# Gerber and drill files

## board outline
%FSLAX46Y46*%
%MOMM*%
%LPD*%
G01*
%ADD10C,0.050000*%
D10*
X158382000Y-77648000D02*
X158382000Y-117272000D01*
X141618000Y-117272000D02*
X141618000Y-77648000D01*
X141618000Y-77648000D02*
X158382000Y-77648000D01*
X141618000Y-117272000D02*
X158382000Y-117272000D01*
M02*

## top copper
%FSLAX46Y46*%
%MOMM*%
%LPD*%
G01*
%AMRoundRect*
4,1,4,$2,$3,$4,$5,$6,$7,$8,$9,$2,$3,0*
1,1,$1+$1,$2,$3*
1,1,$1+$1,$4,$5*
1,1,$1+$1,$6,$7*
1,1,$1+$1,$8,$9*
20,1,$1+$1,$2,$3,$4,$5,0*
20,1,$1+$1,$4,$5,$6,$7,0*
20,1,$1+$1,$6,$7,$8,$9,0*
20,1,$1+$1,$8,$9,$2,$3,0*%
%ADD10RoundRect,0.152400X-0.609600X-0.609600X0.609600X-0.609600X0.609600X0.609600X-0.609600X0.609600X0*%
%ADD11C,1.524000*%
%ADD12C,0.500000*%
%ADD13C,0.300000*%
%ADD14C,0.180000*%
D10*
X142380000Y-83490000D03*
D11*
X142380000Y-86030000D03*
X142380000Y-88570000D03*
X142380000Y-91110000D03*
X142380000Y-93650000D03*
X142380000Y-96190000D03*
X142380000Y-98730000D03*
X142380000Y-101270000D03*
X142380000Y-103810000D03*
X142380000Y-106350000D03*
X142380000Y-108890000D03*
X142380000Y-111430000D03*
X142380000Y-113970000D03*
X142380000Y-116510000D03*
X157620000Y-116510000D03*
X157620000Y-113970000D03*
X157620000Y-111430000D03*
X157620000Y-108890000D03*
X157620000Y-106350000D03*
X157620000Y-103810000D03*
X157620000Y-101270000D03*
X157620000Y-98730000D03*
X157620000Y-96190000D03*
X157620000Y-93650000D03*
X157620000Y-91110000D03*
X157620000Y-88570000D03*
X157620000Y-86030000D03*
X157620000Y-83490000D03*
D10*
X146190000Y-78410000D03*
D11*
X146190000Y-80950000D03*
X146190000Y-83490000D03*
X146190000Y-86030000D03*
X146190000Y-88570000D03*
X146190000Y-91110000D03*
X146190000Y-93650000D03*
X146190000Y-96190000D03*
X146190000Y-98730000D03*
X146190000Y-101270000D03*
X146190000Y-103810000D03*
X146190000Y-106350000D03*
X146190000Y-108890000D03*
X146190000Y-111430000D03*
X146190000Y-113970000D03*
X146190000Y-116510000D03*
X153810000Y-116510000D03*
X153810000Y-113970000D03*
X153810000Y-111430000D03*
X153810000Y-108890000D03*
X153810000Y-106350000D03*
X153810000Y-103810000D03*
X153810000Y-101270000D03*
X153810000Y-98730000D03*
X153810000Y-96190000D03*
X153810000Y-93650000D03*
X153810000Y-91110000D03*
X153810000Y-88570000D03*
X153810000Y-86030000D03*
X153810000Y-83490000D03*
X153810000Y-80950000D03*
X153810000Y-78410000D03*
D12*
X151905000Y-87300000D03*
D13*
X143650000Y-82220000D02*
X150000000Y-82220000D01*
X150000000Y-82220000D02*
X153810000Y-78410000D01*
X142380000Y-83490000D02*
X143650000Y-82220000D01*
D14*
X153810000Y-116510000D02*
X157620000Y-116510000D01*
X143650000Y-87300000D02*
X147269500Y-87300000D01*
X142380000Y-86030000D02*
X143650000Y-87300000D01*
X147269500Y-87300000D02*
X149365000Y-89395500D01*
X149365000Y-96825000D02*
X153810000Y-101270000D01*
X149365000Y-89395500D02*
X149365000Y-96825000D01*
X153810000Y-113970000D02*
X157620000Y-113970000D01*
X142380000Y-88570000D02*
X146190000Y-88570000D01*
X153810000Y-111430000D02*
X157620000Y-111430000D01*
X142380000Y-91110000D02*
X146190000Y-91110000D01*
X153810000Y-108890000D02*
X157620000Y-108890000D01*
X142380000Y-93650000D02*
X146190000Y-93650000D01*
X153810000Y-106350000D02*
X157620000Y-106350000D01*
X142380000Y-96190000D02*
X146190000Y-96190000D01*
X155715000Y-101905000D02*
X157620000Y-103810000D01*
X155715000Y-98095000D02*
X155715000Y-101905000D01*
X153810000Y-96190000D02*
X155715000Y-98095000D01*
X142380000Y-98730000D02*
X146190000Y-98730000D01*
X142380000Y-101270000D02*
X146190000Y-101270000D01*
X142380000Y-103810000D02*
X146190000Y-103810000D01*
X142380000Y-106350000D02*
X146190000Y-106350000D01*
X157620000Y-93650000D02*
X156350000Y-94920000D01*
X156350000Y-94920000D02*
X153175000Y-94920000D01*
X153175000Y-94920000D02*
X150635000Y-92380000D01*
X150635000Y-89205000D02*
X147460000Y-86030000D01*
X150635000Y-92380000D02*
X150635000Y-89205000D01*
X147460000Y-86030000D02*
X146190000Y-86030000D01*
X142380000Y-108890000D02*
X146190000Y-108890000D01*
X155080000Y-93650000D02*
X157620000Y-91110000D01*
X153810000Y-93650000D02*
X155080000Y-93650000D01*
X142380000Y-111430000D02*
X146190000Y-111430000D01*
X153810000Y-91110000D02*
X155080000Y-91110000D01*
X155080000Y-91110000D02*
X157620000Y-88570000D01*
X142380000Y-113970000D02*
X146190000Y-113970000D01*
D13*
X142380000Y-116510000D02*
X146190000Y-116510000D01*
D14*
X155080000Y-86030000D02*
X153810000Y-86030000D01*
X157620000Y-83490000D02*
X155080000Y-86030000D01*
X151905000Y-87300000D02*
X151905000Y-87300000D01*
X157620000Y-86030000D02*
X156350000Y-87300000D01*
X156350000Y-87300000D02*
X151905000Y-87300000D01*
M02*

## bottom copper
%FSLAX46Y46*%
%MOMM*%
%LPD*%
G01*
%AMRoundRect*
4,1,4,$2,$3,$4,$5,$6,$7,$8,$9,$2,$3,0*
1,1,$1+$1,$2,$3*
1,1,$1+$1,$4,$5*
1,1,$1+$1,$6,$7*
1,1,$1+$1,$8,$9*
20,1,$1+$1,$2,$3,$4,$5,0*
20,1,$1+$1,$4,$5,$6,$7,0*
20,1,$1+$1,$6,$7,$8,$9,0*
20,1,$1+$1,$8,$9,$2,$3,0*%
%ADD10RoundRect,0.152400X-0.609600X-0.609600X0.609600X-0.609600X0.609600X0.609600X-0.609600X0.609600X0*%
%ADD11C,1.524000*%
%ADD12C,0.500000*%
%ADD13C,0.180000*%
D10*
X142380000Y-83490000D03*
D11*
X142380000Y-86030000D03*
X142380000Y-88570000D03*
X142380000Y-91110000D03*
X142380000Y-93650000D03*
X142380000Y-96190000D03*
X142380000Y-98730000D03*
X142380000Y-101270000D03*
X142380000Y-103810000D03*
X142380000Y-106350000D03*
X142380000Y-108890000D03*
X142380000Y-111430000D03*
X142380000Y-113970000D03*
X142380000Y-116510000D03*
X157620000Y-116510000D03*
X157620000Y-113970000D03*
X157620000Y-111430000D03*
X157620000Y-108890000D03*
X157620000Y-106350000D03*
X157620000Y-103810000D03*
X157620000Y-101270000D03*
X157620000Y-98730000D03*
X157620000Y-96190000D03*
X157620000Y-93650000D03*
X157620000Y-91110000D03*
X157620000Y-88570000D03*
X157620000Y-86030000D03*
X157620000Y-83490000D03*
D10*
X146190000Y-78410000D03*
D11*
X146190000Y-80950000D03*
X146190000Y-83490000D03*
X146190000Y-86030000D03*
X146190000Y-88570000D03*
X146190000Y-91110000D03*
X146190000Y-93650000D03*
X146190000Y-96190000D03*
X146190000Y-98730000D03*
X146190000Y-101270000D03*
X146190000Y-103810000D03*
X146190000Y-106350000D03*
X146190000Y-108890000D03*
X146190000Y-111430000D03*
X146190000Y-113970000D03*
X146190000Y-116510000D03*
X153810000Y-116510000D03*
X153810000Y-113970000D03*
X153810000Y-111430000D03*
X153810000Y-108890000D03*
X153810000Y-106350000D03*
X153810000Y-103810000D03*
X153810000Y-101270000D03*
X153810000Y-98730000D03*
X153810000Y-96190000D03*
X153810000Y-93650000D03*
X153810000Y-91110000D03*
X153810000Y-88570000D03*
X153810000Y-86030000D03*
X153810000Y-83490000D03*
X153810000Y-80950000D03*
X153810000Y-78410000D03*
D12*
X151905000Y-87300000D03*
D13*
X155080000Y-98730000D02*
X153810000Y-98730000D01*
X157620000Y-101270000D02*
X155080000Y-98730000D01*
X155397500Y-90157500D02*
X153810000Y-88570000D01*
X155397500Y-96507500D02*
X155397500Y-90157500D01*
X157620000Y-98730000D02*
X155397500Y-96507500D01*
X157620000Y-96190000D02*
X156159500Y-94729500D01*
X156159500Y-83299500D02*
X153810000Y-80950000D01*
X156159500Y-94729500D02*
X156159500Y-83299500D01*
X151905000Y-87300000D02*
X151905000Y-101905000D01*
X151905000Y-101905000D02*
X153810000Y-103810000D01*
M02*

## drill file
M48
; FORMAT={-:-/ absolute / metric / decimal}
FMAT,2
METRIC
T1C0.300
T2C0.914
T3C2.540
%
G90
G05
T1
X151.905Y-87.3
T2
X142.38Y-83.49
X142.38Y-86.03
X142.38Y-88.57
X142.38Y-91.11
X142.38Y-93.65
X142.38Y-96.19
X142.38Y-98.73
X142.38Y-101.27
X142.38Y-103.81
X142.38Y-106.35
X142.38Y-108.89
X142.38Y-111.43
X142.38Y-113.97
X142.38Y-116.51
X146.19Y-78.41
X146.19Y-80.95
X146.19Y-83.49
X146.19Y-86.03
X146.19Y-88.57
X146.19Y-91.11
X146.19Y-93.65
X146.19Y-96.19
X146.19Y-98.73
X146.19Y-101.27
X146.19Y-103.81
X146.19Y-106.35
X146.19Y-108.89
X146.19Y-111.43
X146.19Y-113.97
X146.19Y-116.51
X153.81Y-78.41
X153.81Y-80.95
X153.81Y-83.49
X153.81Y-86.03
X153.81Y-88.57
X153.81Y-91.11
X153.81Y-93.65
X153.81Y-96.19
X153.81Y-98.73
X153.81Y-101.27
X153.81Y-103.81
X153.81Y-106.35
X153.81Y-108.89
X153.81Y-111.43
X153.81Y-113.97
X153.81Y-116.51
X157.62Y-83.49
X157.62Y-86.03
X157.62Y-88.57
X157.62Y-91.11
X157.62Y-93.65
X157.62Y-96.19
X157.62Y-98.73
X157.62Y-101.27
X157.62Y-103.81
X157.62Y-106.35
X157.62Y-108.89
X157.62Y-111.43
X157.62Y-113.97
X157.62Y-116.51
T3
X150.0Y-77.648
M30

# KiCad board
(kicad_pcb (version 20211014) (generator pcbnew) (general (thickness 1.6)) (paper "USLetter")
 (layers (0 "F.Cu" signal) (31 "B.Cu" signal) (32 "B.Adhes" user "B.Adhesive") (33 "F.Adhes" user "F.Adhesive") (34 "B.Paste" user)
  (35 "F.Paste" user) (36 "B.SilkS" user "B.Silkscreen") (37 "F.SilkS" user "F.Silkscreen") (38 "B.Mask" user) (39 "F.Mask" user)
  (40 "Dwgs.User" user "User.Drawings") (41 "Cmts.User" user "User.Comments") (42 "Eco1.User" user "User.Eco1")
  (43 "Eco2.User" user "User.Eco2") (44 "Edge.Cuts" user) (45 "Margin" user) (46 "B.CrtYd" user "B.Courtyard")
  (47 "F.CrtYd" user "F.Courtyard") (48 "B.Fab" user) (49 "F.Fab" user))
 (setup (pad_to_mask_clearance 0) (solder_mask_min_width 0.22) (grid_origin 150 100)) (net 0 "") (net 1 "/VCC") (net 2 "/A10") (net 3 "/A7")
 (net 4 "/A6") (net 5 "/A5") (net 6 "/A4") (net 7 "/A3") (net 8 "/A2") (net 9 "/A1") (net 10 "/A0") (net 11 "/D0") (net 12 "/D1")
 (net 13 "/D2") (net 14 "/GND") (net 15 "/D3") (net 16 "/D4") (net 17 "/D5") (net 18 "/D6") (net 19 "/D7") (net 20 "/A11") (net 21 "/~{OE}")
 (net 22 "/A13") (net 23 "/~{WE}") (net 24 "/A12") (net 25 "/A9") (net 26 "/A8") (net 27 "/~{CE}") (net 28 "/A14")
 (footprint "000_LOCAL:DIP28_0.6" (layer "F.Cu") (at 150 100)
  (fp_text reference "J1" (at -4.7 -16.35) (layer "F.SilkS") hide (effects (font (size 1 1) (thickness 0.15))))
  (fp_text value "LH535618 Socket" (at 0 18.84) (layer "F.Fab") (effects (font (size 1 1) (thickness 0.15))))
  (pad "1" thru_hole roundrect locked (at -7.62 -16.51) (size 1.524 1.524) (drill 0.9144) (layers *.Cu *.Mask) (roundrect_rratio 0.1)
   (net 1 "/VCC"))
  (pad "2" thru_hole circle locked (at -7.62 -13.97) (size 1.524 1.524) (drill 0.9144) (layers *.Cu *.Mask) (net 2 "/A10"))
  (pad "3" thru_hole circle locked (at -7.62 -11.43) (size 1.524 1.524) (drill 0.9144) (layers *.Cu *.Mask) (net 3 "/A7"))
  (pad "4" thru_hole circle locked (at -7.62 -8.89) (size 1.524 1.524) (drill 0.9144) (layers *.Cu *.Mask) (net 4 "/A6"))
  (pad "5" thru_hole circle locked (at -7.62 -6.35) (size 1.524 1.524) (drill 0.9144) (layers *.Cu *.Mask) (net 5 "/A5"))
  (pad "6" thru_hole circle locked (at -7.62 -3.81) (size 1.524 1.524) (drill 0.9144) (layers *.Cu *.Mask) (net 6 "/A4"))
  (pad "7" thru_hole circle locked (at -7.62 -1.27) (size 1.524 1.524) (drill 0.9144) (layers *.Cu *.Mask) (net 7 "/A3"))
  (pad "8" thru_hole circle locked (at -7.62 1.27) (size 1.524 1.524) (drill 0.9144) (layers *.Cu *.Mask) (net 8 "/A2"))
  (pad "9" thru_hole circle locked (at -7.62 3.81) (size 1.524 1.524) (drill 0.9144) (layers *.Cu *.Mask) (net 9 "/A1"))
  (pad "10" thru_hole circle locked (at -7.62 6.35) (size 1.524 1.524) (drill 0.9144) (layers *.Cu *.Mask) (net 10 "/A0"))
  (pad "11" thru_hole circle locked (at -7.62 8.89) (size 1.524 1.524) (drill 0.9144) (layers *.Cu *.Mask) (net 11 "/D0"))
  (pad "12" thru_hole circle locked (at -7.62 11.43) (size 1.524 1.524) (drill 0.9144) (layers *.Cu *.Mask) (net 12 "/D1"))
  (pad "13" thru_hole circle locked (at -7.62 13.97) (size 1.524 1.524) (drill 0.9144) (layers *.Cu *.Mask) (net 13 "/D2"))
  (pad "14" thru_hole circle locked (at -7.62 16.51) (size 1.524 1.524) (drill 0.9144) (layers *.Cu *.Mask) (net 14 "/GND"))
  (pad "15" thru_hole circle locked (at 7.62 16.51) (size 1.524 1.524) (drill 0.9144) (layers *.Cu *.Mask) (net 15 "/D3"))
  (pad "16" thru_hole circle locked (at 7.62 13.97) (size 1.524 1.524) (drill 0.9144) (layers *.Cu *.Mask) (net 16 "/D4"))
  (pad "17" thru_hole circle locked (at 7.62 11.43) (size 1.524 1.524) (drill 0.9144) (layers *.Cu *.Mask) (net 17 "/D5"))
  (pad "18" thru_hole circle locked (at 7.62 8.89) (size 1.524 1.524) (drill 0.9144) (layers *.Cu *.Mask) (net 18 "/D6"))
  (pad "19" thru_hole circle locked (at 7.62 6.35) (size 1.524 1.524) (drill 0.9144) (layers *.Cu *.Mask) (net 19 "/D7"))
  (pad "20" thru_hole circle locked (at 7.62 3.81) (size 1.524 1.524) (drill 0.9144) (layers *.Cu *.Mask) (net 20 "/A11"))
  (pad "21" thru_hole circle locked (at 7.62 1.27) (size 1.524 1.524) (drill 0.9144) (layers *.Cu *.Mask) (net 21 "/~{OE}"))
  (pad "22" thru_hole circle locked (at 7.62 -1.27) (size 1.524 1.524) (drill 0.9144) (layers *.Cu *.Mask) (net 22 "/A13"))
  (pad "23" thru_hole circle locked (at 7.62 -3.81) (size 1.524 1.524) (drill 0.9144) (layers *.Cu *.Mask) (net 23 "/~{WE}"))
  (pad "24" thru_hole circle locked (at 7.62 -6.35) (size 1.524 1.524) (drill 0.9144) (layers *.Cu *.Mask) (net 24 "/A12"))
  (pad "25" thru_hole circle locked (at 7.62 -8.89) (size 1.524 1.524) (drill 0.9144) (layers *.Cu *.Mask) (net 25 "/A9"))
  (pad "26" thru_hole circle locked (at 7.62 -11.43) (size 1.524 1.524) (drill 0.9144) (layers *.Cu *.Mask) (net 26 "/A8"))
  (pad "27" thru_hole circle locked (at 7.62 -13.97) (size 1.524 1.524) (drill 0.9144) (layers *.Cu *.Mask) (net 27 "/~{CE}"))
  (pad "28" thru_hole circle locked (at 7.62 -16.51) (size 1.524 1.524) (drill 0.9144) (layers *.Cu *.Mask) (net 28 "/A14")))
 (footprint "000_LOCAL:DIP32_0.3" (layer "F.Cu") (at 150 97.46)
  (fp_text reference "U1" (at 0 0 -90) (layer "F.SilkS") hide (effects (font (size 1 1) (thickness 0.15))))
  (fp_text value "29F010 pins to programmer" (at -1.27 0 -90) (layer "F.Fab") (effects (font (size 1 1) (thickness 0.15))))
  (pad "1" thru_hole roundrect locked (at -3.81 -19.05) (size 1.524 1.524) (drill 0.9144) (layers *.Cu *.Mask) (roundrect_rratio 0.1))
  (pad "2" thru_hole circle locked (at -3.81 -16.51) (size 1.524 1.524) (drill 0.9144) (layers *.Cu *.Mask))
  (pad "3" thru_hole circle locked (at -3.81 -13.97) (size 1.524 1.524) (drill 0.9144) (layers *.Cu *.Mask))
  (pad "4" thru_hole circle locked (at -3.81 -11.43) (size 1.524 1.524) (drill 0.9144) (layers *.Cu *.Mask) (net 24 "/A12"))
  (pad "5" thru_hole circle locked (at -3.81 -8.89) (size 1.524 1.524) (drill 0.9144) (layers *.Cu *.Mask) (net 3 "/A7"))
  (pad "6" thru_hole circle locked (at -3.81 -6.35) (size 1.524 1.524) (drill 0.9144) (layers *.Cu *.Mask) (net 4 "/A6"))
  (pad "7" thru_hole circle locked (at -3.81 -3.81) (size 1.524 1.524) (drill 0.9144) (layers *.Cu *.Mask) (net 5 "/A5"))
  (pad "8" thru_hole circle locked (at -3.81 -1.27) (size 1.524 1.524) (drill 0.9144) (layers *.Cu *.Mask) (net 6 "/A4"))
  (pad "9" thru_hole circle locked (at -3.81 1.27) (size 1.524 1.524) (drill 0.9144) (layers *.Cu *.Mask) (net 7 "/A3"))
  (pad "10" thru_hole circle locked (at -3.81 3.81) (size 1.524 1.524) (drill 0.9144) (layers *.Cu *.Mask) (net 8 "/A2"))
  (pad "11" thru_hole circle locked (at -3.81 6.35) (size 1.524 1.524) (drill 0.9144) (layers *.Cu *.Mask) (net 9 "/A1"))
  (pad "12" thru_hole circle locked (at -3.81 8.89) (size 1.524 1.524) (drill 0.9144) (layers *.Cu *.Mask) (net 10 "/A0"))
  (pad "13" thru_hole circle locked (at -3.81 11.43) (size 1.524 1.524) (drill 0.9144) (layers *.Cu *.Mask) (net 11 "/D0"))
  (pad "14" thru_hole circle locked (at -3.81 13.97) (size 1.524 1.524) (drill 0.9144) (layers *.Cu *.Mask) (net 12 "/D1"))
  (pad "15" thru_hole circle locked (at -3.81 16.51) (size 1.524 1.524) (drill 0.9144) (layers *.Cu *.Mask) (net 13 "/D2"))
  (pad "16" thru_hole circle locked (at -3.81 19.05) (size 1.524 1.524) (drill 0.9144) (layers *.Cu *.Mask) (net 14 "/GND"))
  (pad "17" thru_hole circle locked (at 3.81 19.05) (size 1.524 1.524) (drill 0.9144) (layers *.Cu *.Mask) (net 15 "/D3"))
  (pad "18" thru_hole circle locked (at 3.81 16.51) (size 1.524 1.524) (drill 0.9144) (layers *.Cu *.Mask) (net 16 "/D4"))
  (pad "19" thru_hole circle locked (at 3.81 13.97) (size 1.524 1.524) (drill 0.9144) (layers *.Cu *.Mask) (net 17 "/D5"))
  (pad "20" thru_hole circle locked (at 3.81 11.43) (size 1.524 1.524) (drill 0.9144) (layers *.Cu *.Mask) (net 18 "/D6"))
  (pad "21" thru_hole circle locked (at 3.81 8.89) (size 1.524 1.524) (drill 0.9144) (layers *.Cu *.Mask) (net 19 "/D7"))
  (pad "22" thru_hole circle locked (at 3.81 6.35) (size 1.524 1.524) (drill 0.9144) (layers *.Cu *.Mask) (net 27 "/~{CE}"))
  (pad "23" thru_hole circle locked (at 3.81 3.81) (size 1.524 1.524) (drill 0.9144) (layers *.Cu *.Mask) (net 2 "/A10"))
  (pad "24" thru_hole circle locked (at 3.81 1.27) (size 1.524 1.524) (drill 0.9144) (layers *.Cu *.Mask) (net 21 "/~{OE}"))
  (pad "25" thru_hole circle locked (at 3.81 -1.27) (size 1.524 1.524) (drill 0.9144) (layers *.Cu *.Mask) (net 20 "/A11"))
  (pad "26" thru_hole circle locked (at 3.81 -3.81) (size 1.524 1.524) (drill 0.9144) (layers *.Cu *.Mask) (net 25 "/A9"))
  (pad "27" thru_hole circle locked (at 3.81 -6.35) (size 1.524 1.524) (drill 0.9144) (layers *.Cu *.Mask) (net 26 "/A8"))
  (pad "28" thru_hole circle locked (at 3.81 -8.89) (size 1.524 1.524) (drill 0.9144) (layers *.Cu *.Mask) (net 22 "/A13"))
  (pad "29" thru_hole circle locked (at 3.81 -11.43) (size 1.524 1.524) (drill 0.9144) (layers *.Cu *.Mask) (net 28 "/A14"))
  (pad "30" thru_hole circle locked (at 3.81 -13.97) (size 1.524 1.524) (drill 0.9144) (layers *.Cu *.Mask))
  (pad "31" thru_hole circle locked (at 3.81 -16.51) (size 1.524 1.524) (drill 0.9144) (layers *.Cu *.Mask) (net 23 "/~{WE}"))
  (pad "32" thru_hole circle locked (at 3.81 -19.05) (size 1.524 1.524) (drill 0.9144) (layers *.Cu *.Mask) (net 1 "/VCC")))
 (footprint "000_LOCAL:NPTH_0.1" (layer "F.Cu") (at 150 77.648)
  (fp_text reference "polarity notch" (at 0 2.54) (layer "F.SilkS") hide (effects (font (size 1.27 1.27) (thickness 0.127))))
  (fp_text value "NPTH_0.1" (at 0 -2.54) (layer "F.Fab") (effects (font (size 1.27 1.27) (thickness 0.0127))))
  (pad "" np_thru_hole circle locked (at 0 0) (size 2.54 2.54) (drill 2.54) (layers *.Cu *.Mask)))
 (gr_line (start 158.382 77.648) (end 158.382 117.272) (layer "Edge.Cuts") (width 0.05))
 (gr_line (start 141.618 117.272) (end 141.618 77.648) (layer "Edge.Cuts") (width 0.05))
 (gr_line (start 141.618 77.648) (end 158.382 77.648) (layer "Edge.Cuts") (width 0.05))
 (gr_line (start 141.618 117.272) (end 158.382 117.272) (layer "Edge.Cuts") (width 0.05))
 (segment (start 143.65 82.22) (end 150 82.22) (width 0.3) (layer "F.Cu") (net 1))
 (segment (start 150 82.22) (end 153.81 78.41) (width 0.3) (layer "F.Cu") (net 1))
 (segment (start 142.38 83.49) (end 143.65 82.22) (width 0.3) (layer "F.Cu") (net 1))
 (segment (start 153.81 116.51) (end 157.62 116.51) (width 0.18) (layer "F.Cu") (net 15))
 (segment (start 143.65 87.3) (end 147.2695 87.3) (width 0.18) (layer "F.Cu") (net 2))
 (segment (start 142.38 86.03) (end 143.65 87.3) (width 0.18) (layer "F.Cu") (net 2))
 (segment (start 147.2695 87.3) (end 149.365 89.3955) (width 0.18) (layer "F.Cu") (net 2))
 (segment (start 149.365 96.825) (end 153.81 101.27) (width 0.18) (layer "F.Cu") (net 2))
 (segment (start 149.365 89.3955) (end 149.365 96.825) (width 0.18) (layer "F.Cu") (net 2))
 (segment (start 153.81 113.97) (end 157.62 113.97) (width 0.18) (layer "F.Cu") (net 16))
 (segment (start 142.38 88.57) (end 146.19 88.57) (width 0.18) (layer "F.Cu") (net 3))
 (segment (start 153.81 111.43) (end 157.62 111.43) (width 0.18) (layer "F.Cu") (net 17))
 (segment (start 142.38 91.11) (end 146.19 91.11) (width 0.18) (layer "F.Cu") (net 4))
 (segment (start 153.81 108.89) (end 157.62 108.89) (width 0.18) (layer "F.Cu") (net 18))
 (segment (start 142.38 93.65) (end 146.19 93.65) (width 0.18) (layer "F.Cu") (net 5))
 (segment (start 153.81 106.35) (end 157.62 106.35) (width 0.18) (layer "F.Cu") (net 19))
 (segment (start 142.38 96.19) (end 146.19 96.19) (width 0.18) (layer "F.Cu") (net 6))
 (segment (start 155.715 101.905) (end 157.62 103.81) (width 0.18) (layer "F.Cu") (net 20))
 (segment (start 155.715 98.095) (end 155.715 101.905) (width 0.18) (layer "F.Cu") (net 20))
 (segment (start 153.81 96.19) (end 155.715 98.095) (width 0.18) (layer "F.Cu") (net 20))
 (segment (start 142.38 98.73) (end 146.19 98.73) (width 0.18) (layer "F.Cu") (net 7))
 (segment (start 155.08 98.73) (end 153.81 98.73) (width 0.18) (layer "B.Cu") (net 21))
 (segment (start 157.62 101.27) (end 155.08 98.73) (width 0.18) (layer "B.Cu") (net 21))
 (segment (start 142.38 101.27) (end 146.19 101.27) (width 0.18) (layer "F.Cu") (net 8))
 (segment (start 155.3975 90.1575) (end 153.81 88.57) (width 0.18) (layer "B.Cu") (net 22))
 (segment (start 155.3975 96.5075) (end 155.3975 90.1575) (width 0.18) (layer "B.Cu") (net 22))
 (segment (start 157.62 98.73) (end 155.3975 96.5075) (width 0.18) (layer "B.Cu") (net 22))
 (segment (start 142.38 103.81) (end 146.19 103.81) (width 0.18) (layer "F.Cu") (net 9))
 (segment (start 142.38 106.35) (end 146.19 106.35) (width 0.18) (layer "F.Cu") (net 10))
 (segment (start 157.62 93.65) (end 156.35 94.92) (width 0.18) (layer "F.Cu") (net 24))
 (segment (start 156.35 94.92) (end 153.175 94.92) (width 0.18) (layer "F.Cu") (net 24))
 (segment (start 153.175 94.92) (end 150.635 92.38) (width 0.18) (layer "F.Cu") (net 24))
 (segment (start 150.635 89.205) (end 147.46 86.03) (width 0.18) (layer "F.Cu") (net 24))
 (segment (start 150.635 92.38) (end 150.635 89.205) (width 0.18) (layer "F.Cu") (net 24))
 (segment (start 147.46 86.03) (end 146.19 86.03) (width 0.18) (layer "F.Cu") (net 24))
 (segment (start 142.38 108.89) (end 146.19 108.89) (width 0.18) (layer "F.Cu") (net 11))
 (segment (start 155.08 93.65) (end 157.62 91.11) (width 0.18) (layer "F.Cu") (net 25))
 (segment (start 153.81 93.65) (end 155.08 93.65) (width 0.18) (layer "F.Cu") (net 25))
 (segment (start 142.38 111.43) (end 146.19 111.43) (width 0.18) (layer "F.Cu") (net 12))
 (segment (start 153.81 91.11) (end 155.08 91.11) (width 0.18) (layer "F.Cu") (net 26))
 (segment (start 155.08 91.11) (end 157.62 88.57) (width 0.18) (layer "F.Cu") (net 26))
 (segment (start 142.38 113.97) (end 146.19 113.97) (width 0.18) (layer "F.Cu") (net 13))
 (segment (start 142.38 116.51) (end 146.19 116.51) (width 0.3) (layer "F.Cu") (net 14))
 (segment (start 155.08 86.03) (end 153.81 86.03) (width 0.18) (layer "F.Cu") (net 28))
 (segment (start 157.62 83.49) (end 155.08 86.03) (width 0.18) (layer "F.Cu") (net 28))
 (segment (start 157.62 96.19) (end 156.1595 94.7295) (width 0.18) (layer "B.Cu") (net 23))
 (segment (start 156.1595 83.2995) (end 153.81 80.95) (width 0.18) (layer "B.Cu") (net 23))
 (segment (start 156.1595 94.7295) (end 156.1595 83.2995) (width 0.18) (layer "B.Cu") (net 23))
 (segment (start 151.905 87.3) (end 151.905 87.3) (width 0.18) (layer "F.Cu") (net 27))
 (segment (start 157.62 86.03) (end 156.35 87.3) (width 0.18) (layer "F.Cu") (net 27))
 (segment (start 156.35 87.3) (end 151.905 87.3) (width 0.18) (layer "F.Cu") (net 27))
 (via (at 151.905 87.3) (size 0.5) (drill 0.3) (layers "F.Cu" "B.Cu") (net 27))
 (segment (start 151.905 87.3) (end 151.905 101.905) (width 0.18) (layer "B.Cu") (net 27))
 (segment (start 151.905 101.905) (end 153.81 103.81) (width 0.18) (layer "B.Cu") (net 27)))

